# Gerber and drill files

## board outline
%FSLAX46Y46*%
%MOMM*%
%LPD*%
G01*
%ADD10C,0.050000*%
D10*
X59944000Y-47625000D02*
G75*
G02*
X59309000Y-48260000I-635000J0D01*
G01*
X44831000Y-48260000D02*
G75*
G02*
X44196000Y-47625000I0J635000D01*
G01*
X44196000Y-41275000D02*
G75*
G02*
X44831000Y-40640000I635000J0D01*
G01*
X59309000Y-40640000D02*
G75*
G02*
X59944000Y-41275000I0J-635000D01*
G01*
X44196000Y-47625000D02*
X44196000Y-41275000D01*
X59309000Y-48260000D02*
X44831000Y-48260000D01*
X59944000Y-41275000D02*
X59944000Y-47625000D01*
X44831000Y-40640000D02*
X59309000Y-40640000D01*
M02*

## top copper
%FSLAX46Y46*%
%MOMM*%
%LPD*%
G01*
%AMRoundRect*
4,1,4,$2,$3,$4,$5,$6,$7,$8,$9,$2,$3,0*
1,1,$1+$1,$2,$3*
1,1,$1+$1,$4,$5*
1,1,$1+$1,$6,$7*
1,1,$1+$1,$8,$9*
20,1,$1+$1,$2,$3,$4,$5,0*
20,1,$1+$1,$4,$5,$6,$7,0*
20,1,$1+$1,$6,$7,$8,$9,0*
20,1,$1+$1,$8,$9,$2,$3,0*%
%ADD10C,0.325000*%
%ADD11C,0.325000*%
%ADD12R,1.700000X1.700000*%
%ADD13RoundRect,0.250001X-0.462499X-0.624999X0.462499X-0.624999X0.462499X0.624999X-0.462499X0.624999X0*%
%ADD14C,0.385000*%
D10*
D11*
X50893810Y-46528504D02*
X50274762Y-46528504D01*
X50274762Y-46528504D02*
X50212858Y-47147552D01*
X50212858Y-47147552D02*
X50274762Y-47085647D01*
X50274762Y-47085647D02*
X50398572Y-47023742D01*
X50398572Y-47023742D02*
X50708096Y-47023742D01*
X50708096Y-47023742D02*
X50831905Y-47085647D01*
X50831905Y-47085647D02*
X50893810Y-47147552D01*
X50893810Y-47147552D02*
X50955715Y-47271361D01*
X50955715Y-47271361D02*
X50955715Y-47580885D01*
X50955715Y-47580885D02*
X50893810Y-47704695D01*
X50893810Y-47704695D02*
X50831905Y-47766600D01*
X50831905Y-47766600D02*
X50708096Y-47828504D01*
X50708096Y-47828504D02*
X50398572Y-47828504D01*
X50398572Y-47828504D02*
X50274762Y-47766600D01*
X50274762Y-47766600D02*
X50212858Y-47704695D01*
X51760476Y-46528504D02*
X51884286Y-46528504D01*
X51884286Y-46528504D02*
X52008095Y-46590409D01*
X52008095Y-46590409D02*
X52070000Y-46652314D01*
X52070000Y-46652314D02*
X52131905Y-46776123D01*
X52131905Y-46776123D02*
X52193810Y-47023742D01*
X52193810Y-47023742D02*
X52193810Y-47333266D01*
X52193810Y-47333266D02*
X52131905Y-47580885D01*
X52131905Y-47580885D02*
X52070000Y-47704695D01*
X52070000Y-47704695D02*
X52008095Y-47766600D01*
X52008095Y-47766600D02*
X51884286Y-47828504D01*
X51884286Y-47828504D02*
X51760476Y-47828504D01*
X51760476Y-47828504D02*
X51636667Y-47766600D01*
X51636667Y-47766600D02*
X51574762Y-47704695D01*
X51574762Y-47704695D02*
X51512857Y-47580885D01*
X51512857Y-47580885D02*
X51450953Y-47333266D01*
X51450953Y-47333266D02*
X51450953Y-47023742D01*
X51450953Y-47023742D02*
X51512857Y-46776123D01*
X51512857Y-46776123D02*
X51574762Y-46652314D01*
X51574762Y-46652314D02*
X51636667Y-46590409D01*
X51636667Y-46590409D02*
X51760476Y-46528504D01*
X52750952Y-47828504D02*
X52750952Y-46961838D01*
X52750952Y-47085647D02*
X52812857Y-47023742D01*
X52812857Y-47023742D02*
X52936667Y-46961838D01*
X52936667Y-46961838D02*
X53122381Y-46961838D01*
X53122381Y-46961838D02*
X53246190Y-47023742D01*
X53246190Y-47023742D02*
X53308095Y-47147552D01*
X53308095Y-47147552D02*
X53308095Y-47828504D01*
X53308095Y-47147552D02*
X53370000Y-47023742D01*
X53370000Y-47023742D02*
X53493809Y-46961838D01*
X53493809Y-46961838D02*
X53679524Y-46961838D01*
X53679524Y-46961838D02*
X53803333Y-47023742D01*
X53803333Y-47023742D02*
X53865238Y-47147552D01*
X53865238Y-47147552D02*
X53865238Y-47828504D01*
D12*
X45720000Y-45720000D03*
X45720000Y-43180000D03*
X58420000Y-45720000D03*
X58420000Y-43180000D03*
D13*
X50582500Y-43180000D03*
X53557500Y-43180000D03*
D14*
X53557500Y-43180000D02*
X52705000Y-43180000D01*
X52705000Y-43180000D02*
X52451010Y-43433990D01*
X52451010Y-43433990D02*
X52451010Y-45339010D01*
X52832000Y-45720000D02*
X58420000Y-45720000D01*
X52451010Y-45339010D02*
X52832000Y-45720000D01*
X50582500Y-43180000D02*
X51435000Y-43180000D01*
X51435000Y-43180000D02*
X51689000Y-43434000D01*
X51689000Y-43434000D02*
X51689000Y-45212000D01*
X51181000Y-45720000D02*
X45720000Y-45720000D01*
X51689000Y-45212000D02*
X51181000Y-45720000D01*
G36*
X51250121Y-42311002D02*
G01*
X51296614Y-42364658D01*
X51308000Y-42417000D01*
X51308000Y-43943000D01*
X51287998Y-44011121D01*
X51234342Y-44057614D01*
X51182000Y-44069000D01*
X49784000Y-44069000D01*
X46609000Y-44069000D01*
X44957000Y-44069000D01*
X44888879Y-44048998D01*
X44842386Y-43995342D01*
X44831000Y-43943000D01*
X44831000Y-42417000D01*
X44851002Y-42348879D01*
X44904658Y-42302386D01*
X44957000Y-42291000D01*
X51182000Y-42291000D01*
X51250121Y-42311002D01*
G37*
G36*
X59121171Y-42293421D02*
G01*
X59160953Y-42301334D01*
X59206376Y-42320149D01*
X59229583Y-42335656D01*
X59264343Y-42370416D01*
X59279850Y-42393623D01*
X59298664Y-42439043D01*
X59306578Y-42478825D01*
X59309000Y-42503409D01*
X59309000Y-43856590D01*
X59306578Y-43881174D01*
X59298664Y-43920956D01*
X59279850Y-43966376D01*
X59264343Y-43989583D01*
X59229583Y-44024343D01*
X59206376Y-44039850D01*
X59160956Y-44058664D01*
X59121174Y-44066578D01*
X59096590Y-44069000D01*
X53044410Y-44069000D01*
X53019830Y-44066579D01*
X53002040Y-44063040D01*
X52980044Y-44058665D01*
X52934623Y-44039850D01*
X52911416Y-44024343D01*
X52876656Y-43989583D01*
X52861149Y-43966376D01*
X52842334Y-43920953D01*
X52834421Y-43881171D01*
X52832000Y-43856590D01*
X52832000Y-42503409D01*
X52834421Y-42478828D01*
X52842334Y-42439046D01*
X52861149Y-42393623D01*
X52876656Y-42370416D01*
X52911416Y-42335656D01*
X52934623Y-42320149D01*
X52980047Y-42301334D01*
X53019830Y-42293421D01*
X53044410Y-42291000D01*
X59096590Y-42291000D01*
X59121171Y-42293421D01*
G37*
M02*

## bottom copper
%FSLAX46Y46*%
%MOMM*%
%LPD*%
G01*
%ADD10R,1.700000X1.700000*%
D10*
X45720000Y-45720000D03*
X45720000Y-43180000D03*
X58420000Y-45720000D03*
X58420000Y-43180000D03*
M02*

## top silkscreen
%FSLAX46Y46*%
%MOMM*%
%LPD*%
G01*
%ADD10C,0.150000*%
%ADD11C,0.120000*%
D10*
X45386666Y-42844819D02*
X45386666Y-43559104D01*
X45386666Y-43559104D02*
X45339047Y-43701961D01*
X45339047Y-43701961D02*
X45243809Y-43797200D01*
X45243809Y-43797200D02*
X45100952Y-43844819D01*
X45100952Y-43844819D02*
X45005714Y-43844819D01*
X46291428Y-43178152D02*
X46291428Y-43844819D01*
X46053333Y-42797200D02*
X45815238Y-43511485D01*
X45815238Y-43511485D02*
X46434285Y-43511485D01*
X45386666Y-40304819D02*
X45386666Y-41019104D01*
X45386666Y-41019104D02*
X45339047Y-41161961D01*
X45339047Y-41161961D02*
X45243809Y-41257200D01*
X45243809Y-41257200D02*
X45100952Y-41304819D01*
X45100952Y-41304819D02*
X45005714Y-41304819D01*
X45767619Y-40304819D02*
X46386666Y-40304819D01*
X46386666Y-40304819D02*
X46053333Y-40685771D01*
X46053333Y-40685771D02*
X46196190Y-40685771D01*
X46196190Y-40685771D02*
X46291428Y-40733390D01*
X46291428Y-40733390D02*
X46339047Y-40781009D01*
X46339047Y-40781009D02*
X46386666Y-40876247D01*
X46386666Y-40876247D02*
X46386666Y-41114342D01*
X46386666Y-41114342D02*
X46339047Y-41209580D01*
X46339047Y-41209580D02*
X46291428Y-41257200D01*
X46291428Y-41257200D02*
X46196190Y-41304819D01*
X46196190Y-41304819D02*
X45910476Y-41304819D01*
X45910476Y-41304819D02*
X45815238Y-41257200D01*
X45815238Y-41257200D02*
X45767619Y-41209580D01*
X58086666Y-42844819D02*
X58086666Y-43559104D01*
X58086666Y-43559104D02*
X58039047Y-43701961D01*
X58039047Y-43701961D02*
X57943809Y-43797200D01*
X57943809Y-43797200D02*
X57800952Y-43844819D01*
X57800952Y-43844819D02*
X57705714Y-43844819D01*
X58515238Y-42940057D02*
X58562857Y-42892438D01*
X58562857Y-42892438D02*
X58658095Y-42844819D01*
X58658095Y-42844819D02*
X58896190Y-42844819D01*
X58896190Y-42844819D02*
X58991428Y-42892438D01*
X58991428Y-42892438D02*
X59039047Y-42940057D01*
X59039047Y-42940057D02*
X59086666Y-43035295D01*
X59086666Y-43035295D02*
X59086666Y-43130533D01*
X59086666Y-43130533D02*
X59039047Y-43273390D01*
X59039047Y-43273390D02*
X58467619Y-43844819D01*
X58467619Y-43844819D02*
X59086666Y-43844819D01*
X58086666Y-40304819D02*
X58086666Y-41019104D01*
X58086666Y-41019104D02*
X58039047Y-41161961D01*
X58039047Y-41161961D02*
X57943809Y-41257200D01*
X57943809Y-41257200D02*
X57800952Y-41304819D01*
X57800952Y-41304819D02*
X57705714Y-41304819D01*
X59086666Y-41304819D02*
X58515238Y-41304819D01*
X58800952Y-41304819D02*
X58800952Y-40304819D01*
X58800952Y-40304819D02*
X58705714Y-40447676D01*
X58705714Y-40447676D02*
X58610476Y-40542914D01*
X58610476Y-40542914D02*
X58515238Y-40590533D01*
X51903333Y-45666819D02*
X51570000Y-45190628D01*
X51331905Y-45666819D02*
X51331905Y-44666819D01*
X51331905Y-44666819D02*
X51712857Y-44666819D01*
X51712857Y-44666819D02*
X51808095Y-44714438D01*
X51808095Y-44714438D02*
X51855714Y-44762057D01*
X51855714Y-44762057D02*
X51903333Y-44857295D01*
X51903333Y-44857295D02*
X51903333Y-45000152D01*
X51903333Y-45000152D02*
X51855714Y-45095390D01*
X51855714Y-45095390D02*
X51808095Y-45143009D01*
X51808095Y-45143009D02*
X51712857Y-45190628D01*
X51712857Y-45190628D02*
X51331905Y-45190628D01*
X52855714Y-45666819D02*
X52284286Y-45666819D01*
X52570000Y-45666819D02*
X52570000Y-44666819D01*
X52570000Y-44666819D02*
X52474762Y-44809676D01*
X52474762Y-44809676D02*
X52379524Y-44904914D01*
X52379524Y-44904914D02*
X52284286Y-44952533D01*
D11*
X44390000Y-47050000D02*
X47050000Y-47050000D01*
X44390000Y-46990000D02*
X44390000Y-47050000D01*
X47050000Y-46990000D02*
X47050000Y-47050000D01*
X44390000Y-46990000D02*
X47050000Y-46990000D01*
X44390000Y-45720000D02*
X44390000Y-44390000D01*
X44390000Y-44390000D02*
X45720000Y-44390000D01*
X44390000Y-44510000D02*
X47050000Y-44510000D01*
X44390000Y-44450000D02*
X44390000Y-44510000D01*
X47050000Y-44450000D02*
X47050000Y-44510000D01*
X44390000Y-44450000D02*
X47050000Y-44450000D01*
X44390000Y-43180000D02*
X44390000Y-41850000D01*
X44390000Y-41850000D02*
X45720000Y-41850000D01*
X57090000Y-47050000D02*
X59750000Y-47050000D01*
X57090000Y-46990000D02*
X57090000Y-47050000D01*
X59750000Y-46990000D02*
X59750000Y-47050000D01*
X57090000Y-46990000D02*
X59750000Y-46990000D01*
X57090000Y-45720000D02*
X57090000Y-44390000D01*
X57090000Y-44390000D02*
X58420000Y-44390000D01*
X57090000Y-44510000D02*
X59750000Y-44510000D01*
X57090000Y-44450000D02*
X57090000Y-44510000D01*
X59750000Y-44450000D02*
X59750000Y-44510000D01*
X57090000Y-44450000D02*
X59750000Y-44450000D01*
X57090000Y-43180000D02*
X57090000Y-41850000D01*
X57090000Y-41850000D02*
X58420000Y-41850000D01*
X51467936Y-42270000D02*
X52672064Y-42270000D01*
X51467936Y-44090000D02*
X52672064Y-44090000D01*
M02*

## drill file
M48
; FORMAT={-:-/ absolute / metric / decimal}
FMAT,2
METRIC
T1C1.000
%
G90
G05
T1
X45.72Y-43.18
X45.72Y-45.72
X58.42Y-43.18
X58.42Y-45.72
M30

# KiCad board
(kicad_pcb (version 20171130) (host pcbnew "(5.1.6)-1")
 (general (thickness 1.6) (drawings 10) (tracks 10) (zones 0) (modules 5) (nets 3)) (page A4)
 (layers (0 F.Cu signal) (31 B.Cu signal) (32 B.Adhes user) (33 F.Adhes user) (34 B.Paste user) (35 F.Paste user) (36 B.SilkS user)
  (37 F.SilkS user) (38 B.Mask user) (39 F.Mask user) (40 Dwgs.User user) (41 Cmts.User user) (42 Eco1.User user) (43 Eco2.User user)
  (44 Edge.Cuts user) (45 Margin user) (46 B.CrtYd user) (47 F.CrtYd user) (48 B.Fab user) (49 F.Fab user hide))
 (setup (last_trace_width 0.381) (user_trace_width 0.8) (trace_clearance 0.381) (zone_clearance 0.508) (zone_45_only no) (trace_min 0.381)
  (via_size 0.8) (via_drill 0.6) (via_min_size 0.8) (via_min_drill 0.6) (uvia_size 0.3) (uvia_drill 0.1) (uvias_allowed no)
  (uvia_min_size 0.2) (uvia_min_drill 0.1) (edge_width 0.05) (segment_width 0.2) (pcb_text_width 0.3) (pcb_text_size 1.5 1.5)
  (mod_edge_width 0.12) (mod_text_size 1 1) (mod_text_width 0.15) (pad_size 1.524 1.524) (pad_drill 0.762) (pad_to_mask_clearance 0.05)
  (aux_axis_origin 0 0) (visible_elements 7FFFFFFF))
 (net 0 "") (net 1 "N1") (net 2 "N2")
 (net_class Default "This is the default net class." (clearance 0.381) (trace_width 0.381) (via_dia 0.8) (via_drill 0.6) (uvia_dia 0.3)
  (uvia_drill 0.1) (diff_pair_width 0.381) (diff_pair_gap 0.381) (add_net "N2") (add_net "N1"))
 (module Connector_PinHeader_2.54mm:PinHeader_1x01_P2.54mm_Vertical (layer F.Cu) (at 45.72 45.72)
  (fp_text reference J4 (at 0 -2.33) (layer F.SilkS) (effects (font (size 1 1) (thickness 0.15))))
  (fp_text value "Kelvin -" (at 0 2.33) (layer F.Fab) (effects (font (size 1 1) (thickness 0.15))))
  (fp_line (start -1.33 1.33) (end 1.33 1.33) (layer F.SilkS) (width 0.12))
  (fp_line (start -1.33 1.27) (end -1.33 1.33) (layer F.SilkS) (width 0.12))
  (fp_line (start 1.33 1.27) (end 1.33 1.33) (layer F.SilkS) (width 0.12))
  (fp_line (start -1.33 1.27) (end 1.33 1.27) (layer F.SilkS) (width 0.12))
  (fp_line (start -1.33 0) (end -1.33 -1.33) (layer F.SilkS) (width 0.12))
  (fp_line (start -1.33 -1.33) (end 0 -1.33) (layer F.SilkS) (width 0.12))
  (pad 1 thru_hole rect (at 0 0) (size 1.7 1.7) (drill 1) (layers *.Cu *.Mask) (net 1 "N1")))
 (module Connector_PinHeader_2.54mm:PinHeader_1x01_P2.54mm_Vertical (layer F.Cu) (at 45.72 43.18)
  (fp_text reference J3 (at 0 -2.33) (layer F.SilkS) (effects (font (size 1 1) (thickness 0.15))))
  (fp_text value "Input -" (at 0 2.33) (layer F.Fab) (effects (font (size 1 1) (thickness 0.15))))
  (fp_line (start -1.33 1.33) (end 1.33 1.33) (layer F.SilkS) (width 0.12))
  (fp_line (start -1.33 1.27) (end -1.33 1.33) (layer F.SilkS) (width 0.12))
  (fp_line (start 1.33 1.27) (end 1.33 1.33) (layer F.SilkS) (width 0.12))
  (fp_line (start -1.33 1.27) (end 1.33 1.27) (layer F.SilkS) (width 0.12))
  (fp_line (start -1.33 0) (end -1.33 -1.33) (layer F.SilkS) (width 0.12))
  (fp_line (start -1.33 -1.33) (end 0 -1.33) (layer F.SilkS) (width 0.12))
  (pad 1 thru_hole rect (at 0 0) (size 1.7 1.7) (drill 1) (layers *.Cu *.Mask) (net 1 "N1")))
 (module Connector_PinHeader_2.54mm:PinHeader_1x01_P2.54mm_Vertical (layer F.Cu) (at 58.42 45.72)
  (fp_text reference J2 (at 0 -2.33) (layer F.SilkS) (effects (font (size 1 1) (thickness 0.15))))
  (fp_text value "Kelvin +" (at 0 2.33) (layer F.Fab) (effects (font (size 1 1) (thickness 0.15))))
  (fp_line (start -1.33 1.33) (end 1.33 1.33) (layer F.SilkS) (width 0.12))
  (fp_line (start -1.33 1.27) (end -1.33 1.33) (layer F.SilkS) (width 0.12))
  (fp_line (start 1.33 1.27) (end 1.33 1.33) (layer F.SilkS) (width 0.12))
  (fp_line (start -1.33 1.27) (end 1.33 1.27) (layer F.SilkS) (width 0.12))
  (fp_line (start -1.33 0) (end -1.33 -1.33) (layer F.SilkS) (width 0.12))
  (fp_line (start -1.33 -1.33) (end 0 -1.33) (layer F.SilkS) (width 0.12))
  (pad 1 thru_hole rect (at 0 0) (size 1.7 1.7) (drill 1) (layers *.Cu *.Mask) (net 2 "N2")))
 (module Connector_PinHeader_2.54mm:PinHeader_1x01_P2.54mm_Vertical (layer F.Cu) (at 58.42 43.18)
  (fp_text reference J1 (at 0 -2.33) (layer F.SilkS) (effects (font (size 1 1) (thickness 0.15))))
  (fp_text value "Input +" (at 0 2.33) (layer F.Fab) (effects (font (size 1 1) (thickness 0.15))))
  (fp_line (start -1.33 1.33) (end 1.33 1.33) (layer F.SilkS) (width 0.12))
  (fp_line (start -1.33 1.27) (end -1.33 1.33) (layer F.SilkS) (width 0.12))
  (fp_line (start 1.33 1.27) (end 1.33 1.33) (layer F.SilkS) (width 0.12))
  (fp_line (start -1.33 1.27) (end 1.33 1.27) (layer F.SilkS) (width 0.12))
  (fp_line (start -1.33 0) (end -1.33 -1.33) (layer F.SilkS) (width 0.12))
  (fp_line (start -1.33 -1.33) (end 0 -1.33) (layer F.SilkS) (width 0.12))
  (pad 1 thru_hole rect (at 0 0) (size 1.7 1.7) (drill 1) (layers *.Cu *.Mask) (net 2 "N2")))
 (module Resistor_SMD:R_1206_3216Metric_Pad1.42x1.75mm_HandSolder (layer F.Cu) (at 52.07 43.18)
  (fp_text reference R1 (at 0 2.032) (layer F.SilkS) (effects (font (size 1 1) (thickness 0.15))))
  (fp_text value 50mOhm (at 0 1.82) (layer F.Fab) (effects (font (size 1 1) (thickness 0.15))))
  (fp_line (start -0.602064 -0.91) (end 0.602064 -0.91) (layer F.SilkS) (width 0.12))
  (fp_line (start -0.602064 0.91) (end 0.602064 0.91) (layer F.SilkS) (width 0.12))
  (pad 1 smd roundrect (at -1.4875 0) (size 1.425 1.75) (layers F.Cu F.Paste F.Mask) (roundrect_rratio 0.175439) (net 1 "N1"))
  (pad 2 smd roundrect (at 1.4875 0) (size 1.425 1.75) (layers F.Cu F.Paste F.Mask) (roundrect_rratio 0.175439) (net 2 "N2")))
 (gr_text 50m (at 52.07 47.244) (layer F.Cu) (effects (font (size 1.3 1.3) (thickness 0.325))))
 (gr_arc (start 59.309 47.625) (end 59.309 48.26) (angle -90) (layer Edge.Cuts) (width 0.05))
 (gr_arc (start 44.831 47.625) (end 44.196 47.625) (angle -90) (layer Edge.Cuts) (width 0.05))
 (gr_arc (start 44.831 41.275) (end 44.831 40.64) (angle -90) (layer Edge.Cuts) (width 0.05))
 (gr_arc (start 59.309 41.275) (end 59.944 41.275) (angle -90) (layer Edge.Cuts) (width 0.05))
 (gr_line (start 44.196 47.625) (end 44.196 41.275) (layer Edge.Cuts) (width 0.05))
 (gr_line (start 59.309 48.26) (end 44.831 48.26) (layer Edge.Cuts) (width 0.05))
 (gr_line (start 59.944 41.275) (end 59.944 47.625) (layer Edge.Cuts) (width 0.05))
 (gr_line (start 44.831 40.64) (end 59.309 40.64) (layer Edge.Cuts) (width 0.05))
 (segment (start 53.5575 43.18) (end 52.705 43.18) (width 0.385) (layer F.Cu) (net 2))
 (segment (start 52.705 43.18) (end 52.45101 43.43399) (width 0.385) (layer F.Cu) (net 2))
 (segment (start 52.45101 43.43399) (end 52.45101 45.33901) (width 0.385) (layer F.Cu) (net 2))
 (segment (start 52.832 45.72) (end 58.42 45.72) (width 0.385) (layer F.Cu) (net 2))
 (segment (start 52.45101 45.33901) (end 52.832 45.72) (width 0.385) (layer F.Cu) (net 2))
 (segment (start 50.5825 43.18) (end 51.435 43.18) (width 0.385) (layer F.Cu) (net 1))
 (segment (start 51.435 43.18) (end 51.689 43.434) (width 0.385) (layer F.Cu) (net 1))
 (segment (start 51.689 43.434) (end 51.689 45.212) (width 0.385) (layer F.Cu) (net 1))
 (segment (start 51.181 45.72) (end 45.72 45.72) (width 0.385) (layer F.Cu) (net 1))
 (segment (start 51.689 45.212) (end 51.181 45.72) (width 0.385) (layer F.Cu) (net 1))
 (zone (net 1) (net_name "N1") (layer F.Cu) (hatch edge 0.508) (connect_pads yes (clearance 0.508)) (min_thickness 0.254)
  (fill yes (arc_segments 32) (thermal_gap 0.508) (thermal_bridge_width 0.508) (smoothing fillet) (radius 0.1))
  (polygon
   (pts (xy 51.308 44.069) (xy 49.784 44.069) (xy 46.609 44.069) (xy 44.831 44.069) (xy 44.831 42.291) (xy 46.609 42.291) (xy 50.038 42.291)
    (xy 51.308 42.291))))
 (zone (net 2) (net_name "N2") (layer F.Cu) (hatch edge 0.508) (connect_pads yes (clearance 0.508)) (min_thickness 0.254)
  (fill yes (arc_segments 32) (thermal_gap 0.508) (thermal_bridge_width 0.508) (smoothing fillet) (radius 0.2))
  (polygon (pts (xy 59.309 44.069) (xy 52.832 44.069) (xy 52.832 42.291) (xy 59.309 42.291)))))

